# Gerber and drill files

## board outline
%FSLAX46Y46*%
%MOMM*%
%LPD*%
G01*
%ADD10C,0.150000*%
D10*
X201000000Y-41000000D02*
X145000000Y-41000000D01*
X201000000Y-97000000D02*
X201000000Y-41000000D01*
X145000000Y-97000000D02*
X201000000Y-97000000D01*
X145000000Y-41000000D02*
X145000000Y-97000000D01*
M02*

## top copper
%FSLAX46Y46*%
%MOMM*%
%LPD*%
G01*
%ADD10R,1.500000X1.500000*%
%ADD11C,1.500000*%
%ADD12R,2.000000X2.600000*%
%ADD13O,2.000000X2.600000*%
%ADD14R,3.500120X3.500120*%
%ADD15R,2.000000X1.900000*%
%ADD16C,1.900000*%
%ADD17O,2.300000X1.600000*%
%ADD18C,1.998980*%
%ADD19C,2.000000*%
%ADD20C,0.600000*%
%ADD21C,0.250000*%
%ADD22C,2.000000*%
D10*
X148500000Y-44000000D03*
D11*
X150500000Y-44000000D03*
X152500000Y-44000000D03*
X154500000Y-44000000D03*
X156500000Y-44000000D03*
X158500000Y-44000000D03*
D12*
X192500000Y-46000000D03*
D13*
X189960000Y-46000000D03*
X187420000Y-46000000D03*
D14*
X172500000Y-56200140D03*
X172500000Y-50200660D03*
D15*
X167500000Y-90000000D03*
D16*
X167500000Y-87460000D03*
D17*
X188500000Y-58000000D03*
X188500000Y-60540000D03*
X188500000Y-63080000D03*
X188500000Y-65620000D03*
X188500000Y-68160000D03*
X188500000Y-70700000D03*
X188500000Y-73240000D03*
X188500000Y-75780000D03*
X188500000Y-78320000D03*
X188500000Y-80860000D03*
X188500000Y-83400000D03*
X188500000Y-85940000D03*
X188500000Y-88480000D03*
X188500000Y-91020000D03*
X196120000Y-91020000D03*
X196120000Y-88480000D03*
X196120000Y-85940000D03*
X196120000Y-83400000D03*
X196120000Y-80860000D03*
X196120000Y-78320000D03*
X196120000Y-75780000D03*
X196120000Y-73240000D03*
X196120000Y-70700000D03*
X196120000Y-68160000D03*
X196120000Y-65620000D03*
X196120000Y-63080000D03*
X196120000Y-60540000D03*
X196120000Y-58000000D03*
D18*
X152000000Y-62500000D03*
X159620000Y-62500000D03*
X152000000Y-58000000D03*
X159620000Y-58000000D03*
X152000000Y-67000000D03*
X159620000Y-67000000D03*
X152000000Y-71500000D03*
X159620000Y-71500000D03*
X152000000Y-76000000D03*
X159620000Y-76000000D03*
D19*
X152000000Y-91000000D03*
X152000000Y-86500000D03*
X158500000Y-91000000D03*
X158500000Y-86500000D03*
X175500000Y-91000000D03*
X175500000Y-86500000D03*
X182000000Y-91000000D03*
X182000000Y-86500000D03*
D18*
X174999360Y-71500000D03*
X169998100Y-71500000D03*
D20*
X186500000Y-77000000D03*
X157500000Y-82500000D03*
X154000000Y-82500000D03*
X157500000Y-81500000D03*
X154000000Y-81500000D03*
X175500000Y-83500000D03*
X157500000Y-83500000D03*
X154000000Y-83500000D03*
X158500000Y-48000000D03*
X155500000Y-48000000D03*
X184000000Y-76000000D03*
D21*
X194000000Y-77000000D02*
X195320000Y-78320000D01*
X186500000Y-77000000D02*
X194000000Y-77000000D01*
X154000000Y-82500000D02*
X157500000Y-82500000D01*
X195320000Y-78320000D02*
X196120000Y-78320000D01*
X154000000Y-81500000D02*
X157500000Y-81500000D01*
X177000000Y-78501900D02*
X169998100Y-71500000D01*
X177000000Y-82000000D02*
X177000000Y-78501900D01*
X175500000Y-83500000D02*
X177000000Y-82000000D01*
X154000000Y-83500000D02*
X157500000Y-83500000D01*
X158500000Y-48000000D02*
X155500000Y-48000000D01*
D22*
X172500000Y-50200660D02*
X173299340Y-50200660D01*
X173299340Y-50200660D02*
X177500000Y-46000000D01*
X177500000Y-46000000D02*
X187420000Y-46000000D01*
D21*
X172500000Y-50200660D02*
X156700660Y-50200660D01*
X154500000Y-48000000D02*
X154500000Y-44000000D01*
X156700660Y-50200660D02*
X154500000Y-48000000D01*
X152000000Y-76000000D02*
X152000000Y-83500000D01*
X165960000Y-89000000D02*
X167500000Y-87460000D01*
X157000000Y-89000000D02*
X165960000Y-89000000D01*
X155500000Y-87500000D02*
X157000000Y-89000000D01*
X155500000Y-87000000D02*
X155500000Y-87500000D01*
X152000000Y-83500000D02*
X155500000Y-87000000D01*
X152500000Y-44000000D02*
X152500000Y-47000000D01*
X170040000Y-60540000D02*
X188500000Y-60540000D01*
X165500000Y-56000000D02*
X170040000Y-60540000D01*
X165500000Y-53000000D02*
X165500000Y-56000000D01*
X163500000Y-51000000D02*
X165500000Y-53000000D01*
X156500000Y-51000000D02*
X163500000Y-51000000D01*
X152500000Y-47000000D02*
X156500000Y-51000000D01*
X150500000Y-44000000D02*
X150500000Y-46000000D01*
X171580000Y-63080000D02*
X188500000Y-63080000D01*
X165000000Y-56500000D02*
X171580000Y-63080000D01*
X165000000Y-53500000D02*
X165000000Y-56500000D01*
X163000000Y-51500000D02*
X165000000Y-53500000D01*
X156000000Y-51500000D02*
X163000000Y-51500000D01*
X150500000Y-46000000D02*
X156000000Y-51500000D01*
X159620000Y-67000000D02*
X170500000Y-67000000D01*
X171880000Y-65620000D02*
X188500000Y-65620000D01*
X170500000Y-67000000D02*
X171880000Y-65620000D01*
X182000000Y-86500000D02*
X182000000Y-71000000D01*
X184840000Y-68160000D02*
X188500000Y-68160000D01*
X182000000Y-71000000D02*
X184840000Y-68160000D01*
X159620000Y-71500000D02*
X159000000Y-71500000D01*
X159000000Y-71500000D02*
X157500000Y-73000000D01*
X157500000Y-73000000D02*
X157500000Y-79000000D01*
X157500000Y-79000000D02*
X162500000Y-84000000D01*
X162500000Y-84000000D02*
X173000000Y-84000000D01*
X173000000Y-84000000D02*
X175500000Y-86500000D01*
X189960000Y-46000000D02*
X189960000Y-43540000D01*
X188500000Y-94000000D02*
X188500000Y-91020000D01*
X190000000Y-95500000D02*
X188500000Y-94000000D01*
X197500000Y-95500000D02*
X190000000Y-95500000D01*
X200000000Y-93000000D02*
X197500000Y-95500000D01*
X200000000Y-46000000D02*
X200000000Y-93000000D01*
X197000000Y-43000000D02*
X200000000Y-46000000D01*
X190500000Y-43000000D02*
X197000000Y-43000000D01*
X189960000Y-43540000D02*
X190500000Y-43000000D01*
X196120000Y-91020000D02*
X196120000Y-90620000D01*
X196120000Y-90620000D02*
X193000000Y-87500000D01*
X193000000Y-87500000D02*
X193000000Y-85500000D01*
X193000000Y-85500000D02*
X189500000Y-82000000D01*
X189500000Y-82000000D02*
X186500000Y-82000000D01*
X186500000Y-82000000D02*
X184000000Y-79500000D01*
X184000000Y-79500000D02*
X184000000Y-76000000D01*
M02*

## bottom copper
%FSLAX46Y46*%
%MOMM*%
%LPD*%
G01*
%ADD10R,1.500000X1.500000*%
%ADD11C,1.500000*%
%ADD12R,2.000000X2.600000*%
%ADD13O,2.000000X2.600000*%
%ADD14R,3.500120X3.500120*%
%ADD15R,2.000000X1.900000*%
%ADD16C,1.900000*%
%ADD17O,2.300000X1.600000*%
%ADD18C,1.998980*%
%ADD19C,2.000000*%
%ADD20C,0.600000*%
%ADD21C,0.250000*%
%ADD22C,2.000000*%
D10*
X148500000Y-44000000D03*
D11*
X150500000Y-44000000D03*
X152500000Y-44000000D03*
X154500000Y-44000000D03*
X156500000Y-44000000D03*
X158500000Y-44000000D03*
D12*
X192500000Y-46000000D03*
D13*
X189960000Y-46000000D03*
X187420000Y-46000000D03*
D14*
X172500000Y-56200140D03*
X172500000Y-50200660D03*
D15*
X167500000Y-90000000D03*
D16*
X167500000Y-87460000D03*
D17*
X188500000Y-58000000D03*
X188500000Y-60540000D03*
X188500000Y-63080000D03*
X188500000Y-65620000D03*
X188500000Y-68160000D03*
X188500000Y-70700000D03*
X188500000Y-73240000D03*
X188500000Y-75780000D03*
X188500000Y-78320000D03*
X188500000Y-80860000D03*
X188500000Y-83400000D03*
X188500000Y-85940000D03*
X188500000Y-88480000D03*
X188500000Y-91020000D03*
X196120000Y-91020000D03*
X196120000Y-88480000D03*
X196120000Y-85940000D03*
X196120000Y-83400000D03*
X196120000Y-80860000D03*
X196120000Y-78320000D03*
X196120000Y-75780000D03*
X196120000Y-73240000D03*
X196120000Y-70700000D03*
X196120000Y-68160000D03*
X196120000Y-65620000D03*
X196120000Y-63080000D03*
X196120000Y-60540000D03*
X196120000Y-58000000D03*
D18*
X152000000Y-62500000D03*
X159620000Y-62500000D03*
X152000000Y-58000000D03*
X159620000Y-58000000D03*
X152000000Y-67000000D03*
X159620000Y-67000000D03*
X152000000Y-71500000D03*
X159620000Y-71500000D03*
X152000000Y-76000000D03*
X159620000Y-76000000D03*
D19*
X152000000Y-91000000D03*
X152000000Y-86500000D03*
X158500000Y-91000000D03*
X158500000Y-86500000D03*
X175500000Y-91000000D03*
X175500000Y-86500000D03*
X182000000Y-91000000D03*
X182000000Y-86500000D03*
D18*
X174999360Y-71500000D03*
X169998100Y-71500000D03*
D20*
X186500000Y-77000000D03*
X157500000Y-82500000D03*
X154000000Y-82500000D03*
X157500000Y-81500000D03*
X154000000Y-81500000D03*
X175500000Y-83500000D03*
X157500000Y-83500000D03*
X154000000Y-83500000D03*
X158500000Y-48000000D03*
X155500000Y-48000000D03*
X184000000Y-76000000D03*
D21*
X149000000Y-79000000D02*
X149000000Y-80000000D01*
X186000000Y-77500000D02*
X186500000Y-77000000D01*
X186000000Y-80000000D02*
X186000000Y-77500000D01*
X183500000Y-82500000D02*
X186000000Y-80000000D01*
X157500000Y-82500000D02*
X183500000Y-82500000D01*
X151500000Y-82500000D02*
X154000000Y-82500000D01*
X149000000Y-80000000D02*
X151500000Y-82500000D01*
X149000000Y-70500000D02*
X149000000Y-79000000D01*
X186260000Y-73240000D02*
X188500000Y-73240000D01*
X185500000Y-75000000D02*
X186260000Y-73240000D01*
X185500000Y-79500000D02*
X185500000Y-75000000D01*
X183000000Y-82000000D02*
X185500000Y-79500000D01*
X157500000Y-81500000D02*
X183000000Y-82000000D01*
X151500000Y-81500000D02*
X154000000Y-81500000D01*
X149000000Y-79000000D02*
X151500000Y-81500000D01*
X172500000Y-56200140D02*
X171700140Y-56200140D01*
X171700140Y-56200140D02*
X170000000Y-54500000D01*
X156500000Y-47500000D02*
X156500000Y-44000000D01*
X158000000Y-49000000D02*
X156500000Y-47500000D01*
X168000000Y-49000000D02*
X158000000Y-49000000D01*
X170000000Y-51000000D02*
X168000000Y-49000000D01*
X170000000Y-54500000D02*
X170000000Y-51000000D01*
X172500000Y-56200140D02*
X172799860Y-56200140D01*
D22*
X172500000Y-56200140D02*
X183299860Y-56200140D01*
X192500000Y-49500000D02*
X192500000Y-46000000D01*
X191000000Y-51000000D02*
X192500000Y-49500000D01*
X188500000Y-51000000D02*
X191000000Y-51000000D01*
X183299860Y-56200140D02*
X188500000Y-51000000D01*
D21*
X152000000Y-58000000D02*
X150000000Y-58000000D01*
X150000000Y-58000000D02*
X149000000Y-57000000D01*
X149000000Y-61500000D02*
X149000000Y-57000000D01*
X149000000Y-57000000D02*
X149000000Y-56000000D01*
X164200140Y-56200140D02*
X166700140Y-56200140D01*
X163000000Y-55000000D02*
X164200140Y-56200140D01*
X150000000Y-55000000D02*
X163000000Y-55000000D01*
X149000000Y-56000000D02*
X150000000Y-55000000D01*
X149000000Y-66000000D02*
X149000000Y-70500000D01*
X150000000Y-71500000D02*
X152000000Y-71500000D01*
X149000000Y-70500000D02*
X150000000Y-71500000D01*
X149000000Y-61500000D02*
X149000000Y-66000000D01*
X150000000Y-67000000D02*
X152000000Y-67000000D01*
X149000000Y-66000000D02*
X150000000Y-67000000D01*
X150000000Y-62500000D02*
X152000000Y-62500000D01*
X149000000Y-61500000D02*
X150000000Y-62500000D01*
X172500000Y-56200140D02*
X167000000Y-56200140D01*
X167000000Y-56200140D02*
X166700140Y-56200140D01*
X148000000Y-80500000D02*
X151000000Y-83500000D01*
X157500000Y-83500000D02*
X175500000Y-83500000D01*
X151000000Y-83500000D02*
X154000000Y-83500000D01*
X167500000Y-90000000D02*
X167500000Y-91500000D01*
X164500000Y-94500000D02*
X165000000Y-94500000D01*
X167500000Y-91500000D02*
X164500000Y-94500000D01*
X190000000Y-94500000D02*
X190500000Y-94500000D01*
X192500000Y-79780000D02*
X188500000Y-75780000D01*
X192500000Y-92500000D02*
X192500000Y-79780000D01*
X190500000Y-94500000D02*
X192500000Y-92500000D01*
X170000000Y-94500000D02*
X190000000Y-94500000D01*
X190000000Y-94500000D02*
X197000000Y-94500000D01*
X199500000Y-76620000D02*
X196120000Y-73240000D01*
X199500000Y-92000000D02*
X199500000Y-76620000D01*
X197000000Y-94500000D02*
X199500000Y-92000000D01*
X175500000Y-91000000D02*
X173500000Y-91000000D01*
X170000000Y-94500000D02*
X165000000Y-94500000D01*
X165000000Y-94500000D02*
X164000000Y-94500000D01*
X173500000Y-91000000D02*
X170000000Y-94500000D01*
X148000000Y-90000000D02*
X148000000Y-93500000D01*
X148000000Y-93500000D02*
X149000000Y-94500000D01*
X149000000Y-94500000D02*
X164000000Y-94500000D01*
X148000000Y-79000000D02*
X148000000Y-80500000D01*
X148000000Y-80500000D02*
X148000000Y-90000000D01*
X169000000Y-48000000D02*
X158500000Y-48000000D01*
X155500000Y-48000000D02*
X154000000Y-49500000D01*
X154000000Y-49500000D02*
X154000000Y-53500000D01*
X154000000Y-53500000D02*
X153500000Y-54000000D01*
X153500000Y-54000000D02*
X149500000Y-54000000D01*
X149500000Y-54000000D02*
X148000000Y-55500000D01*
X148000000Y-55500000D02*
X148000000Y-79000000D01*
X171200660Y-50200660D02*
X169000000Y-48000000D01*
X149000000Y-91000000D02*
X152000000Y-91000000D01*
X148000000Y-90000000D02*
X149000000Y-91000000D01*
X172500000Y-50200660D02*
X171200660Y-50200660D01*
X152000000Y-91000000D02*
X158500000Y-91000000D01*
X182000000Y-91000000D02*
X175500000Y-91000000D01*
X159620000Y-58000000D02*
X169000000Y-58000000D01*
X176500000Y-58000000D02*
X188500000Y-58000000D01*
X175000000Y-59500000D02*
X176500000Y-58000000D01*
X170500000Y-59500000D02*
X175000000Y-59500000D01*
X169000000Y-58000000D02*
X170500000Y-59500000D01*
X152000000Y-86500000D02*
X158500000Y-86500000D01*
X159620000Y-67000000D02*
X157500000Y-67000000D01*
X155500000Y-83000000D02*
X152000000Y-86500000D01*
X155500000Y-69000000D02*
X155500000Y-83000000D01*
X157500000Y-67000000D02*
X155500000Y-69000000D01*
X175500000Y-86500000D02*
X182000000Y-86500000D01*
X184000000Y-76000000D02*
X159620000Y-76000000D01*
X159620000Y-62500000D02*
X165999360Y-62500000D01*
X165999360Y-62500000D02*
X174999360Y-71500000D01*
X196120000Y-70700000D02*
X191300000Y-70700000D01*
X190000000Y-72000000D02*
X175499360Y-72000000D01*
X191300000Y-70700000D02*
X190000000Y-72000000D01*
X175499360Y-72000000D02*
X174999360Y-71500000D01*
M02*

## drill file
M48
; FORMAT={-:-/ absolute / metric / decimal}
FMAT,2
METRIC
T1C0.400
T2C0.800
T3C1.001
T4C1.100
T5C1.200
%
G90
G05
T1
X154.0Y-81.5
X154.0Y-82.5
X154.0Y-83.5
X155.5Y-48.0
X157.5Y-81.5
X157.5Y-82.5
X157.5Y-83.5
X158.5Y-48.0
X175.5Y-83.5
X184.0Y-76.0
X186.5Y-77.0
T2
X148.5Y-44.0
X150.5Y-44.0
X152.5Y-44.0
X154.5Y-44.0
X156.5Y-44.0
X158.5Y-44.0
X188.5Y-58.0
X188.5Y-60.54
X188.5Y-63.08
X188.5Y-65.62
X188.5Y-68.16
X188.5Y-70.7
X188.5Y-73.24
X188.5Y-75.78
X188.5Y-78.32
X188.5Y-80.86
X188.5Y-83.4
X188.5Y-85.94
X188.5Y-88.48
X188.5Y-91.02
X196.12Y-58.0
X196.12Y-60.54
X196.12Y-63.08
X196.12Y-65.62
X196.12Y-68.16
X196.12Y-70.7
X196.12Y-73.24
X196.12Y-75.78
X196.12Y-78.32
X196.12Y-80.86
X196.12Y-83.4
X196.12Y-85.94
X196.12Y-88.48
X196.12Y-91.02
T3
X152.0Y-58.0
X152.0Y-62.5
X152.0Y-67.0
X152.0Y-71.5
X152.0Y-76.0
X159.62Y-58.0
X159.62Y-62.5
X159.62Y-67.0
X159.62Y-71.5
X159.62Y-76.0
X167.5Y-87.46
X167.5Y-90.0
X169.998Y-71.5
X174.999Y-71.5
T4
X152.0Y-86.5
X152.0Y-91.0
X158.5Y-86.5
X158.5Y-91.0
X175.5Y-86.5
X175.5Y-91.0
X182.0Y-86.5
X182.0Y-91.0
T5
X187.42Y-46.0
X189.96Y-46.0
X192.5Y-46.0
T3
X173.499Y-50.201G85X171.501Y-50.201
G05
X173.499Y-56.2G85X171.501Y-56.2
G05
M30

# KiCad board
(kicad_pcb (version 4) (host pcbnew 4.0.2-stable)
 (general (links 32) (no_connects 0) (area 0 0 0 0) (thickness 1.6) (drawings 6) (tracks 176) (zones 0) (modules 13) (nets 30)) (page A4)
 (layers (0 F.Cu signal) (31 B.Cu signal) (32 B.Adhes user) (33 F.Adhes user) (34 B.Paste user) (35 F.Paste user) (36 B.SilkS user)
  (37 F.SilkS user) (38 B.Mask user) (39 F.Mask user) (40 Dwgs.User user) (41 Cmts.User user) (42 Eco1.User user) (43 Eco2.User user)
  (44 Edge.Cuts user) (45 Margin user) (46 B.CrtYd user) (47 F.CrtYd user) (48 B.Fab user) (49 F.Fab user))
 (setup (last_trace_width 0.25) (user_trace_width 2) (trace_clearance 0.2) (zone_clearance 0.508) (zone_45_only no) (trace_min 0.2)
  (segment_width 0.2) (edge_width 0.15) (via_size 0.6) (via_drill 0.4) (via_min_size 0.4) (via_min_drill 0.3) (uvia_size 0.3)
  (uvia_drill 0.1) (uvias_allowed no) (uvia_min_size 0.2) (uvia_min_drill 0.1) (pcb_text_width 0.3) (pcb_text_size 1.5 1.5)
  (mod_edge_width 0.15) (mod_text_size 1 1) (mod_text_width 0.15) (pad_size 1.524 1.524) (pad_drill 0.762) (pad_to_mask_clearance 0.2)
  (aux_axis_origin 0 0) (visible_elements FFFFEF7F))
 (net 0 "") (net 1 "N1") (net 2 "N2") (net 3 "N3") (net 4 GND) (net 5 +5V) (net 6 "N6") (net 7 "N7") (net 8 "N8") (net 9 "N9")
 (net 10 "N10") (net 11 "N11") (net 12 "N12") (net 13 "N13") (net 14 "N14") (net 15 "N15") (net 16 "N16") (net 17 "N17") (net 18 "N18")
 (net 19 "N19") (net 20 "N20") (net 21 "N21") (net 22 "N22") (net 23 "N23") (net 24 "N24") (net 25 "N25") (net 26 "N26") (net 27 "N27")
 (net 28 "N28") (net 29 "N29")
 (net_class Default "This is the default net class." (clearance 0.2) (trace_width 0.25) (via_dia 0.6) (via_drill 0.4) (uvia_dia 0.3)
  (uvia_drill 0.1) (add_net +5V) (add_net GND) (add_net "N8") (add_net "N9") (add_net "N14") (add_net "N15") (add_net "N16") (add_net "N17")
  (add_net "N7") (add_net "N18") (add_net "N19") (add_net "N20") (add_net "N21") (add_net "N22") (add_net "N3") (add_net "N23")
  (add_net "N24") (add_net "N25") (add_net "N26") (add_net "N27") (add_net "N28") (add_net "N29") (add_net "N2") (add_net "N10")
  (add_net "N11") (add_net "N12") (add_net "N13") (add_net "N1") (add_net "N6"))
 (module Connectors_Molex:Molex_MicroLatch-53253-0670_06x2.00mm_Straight (layer F.Cu) (at 148.5 44)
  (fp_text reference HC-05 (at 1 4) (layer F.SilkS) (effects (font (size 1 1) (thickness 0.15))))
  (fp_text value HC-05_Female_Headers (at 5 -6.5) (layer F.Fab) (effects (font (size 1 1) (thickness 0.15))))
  (pad 1 thru_hole rect (at 0 0) (size 1.5 1.5) (drill 0.8) (layers *.Cu *.Mask) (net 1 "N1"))
  (pad 2 thru_hole circle (at 2 0) (size 1.5 1.5) (drill 0.8) (layers *.Cu *.Mask) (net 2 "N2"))
  (pad 3 thru_hole circle (at 4 0) (size 1.5 1.5) (drill 0.8) (layers *.Cu *.Mask) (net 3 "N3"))
  (pad 4 thru_hole circle (at 6 0) (size 1.5 1.5) (drill 0.8) (layers *.Cu *.Mask) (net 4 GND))
  (pad 5 thru_hole circle (at 8 0) (size 1.5 1.5) (drill 0.8) (layers *.Cu *.Mask) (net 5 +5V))
  (pad 6 thru_hole circle (at 10 0) (size 1.5 1.5) (drill 0.8) (layers *.Cu *.Mask) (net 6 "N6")))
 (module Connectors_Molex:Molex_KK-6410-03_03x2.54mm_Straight (layer F.Cu) (at 192.5 46 180)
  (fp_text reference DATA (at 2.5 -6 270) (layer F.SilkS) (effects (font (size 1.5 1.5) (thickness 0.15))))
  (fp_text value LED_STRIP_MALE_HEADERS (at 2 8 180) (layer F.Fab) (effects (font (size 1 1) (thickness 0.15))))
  (pad 1 thru_hole rect (at 0 0 180) (size 2 2.6) (drill 1.2) (layers *.Cu *.Mask F.SilkS) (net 5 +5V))
  (pad 2 thru_hole oval (at 2.54 0 180) (size 2 2.6) (drill 1.2) (layers *.Cu *.Mask F.SilkS) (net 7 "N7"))
  (pad 3 thru_hole oval (at 5.08 0 180) (size 2 2.6) (drill 1.2) (layers *.Cu *.Mask F.SilkS) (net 4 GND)))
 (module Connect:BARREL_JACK (layer F.Cu) (at 172.5 50 270)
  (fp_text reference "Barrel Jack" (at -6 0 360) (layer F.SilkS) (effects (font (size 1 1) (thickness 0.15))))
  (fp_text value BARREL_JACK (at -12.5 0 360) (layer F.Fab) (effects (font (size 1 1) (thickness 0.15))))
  (pad 1 thru_hole rect (at 6.20014 0 270) (size 3.50012 3.50012) (drill oval 1.00076 2.99974) (layers *.Cu *.Mask F.SilkS) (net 5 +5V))
  (pad 2 thru_hole rect (at 0.20066 0 270) (size 3.50012 3.50012) (drill oval 1.00076 2.99974) (layers *.Cu *.Mask F.SilkS) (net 4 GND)))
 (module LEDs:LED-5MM (layer F.Cu) (at 167.5 90 90)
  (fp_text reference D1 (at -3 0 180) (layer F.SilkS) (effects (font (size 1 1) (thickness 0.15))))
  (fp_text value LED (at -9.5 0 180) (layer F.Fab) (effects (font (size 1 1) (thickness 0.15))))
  (pad 1 thru_hole rect (at 0 0 180) (size 2 1.9) (drill 1.00076) (layers *.Cu *.Mask F.SilkS) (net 4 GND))
  (pad 2 thru_hole circle (at 2.54 0 90) (size 1.9 1.9) (drill 1.00076) (layers *.Cu *.Mask F.SilkS) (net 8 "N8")))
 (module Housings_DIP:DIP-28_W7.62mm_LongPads (layer F.Cu) (at 188.5 58)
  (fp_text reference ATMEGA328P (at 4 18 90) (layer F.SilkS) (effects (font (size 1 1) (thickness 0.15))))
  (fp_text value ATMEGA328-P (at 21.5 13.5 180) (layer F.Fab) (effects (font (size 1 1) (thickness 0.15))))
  (pad 1 thru_hole oval (at 0 0) (size 2.3 1.6) (drill 0.8) (layers *.Cu *.Mask F.SilkS) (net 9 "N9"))
  (pad 2 thru_hole oval (at 0 2.54) (size 2.3 1.6) (drill 0.8) (layers *.Cu *.Mask F.SilkS) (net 3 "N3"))
  (pad 3 thru_hole oval (at 0 5.08) (size 2.3 1.6) (drill 0.8) (layers *.Cu *.Mask F.SilkS) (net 2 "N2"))
  (pad 4 thru_hole oval (at 0 7.62) (size 2.3 1.6) (drill 0.8) (layers *.Cu *.Mask F.SilkS) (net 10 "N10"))
  (pad 5 thru_hole oval (at 0 10.16) (size 2.3 1.6) (drill 0.8) (layers *.Cu *.Mask F.SilkS) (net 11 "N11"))
  (pad 6 thru_hole oval (at 0 12.7) (size 2.3 1.6) (drill 0.8) (layers *.Cu *.Mask F.SilkS) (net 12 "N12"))
  (pad 7 thru_hole oval (at 0 15.24) (size 2.3 1.6) (drill 0.8) (layers *.Cu *.Mask F.SilkS) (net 5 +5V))
  (pad 8 thru_hole oval (at 0 17.78) (size 2.3 1.6) (drill 0.8) (layers *.Cu *.Mask F.SilkS) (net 4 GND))
  (pad 9 thru_hole oval (at 0 20.32) (size 2.3 1.6) (drill 0.8) (layers *.Cu *.Mask F.SilkS) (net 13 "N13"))
  (pad 10 thru_hole oval (at 0 22.86) (size 2.3 1.6) (drill 0.8) (layers *.Cu *.Mask F.SilkS) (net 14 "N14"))
  (pad 11 thru_hole oval (at 0 25.4) (size 2.3 1.6) (drill 0.8) (layers *.Cu *.Mask F.SilkS) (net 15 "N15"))
  (pad 12 thru_hole oval (at 0 27.94) (size 2.3 1.6) (drill 0.8) (layers *.Cu *.Mask F.SilkS) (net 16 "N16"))
  (pad 13 thru_hole oval (at 0 30.48) (size 2.3 1.6) (drill 0.8) (layers *.Cu *.Mask F.SilkS) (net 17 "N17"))
  (pad 14 thru_hole oval (at 0 33.02) (size 2.3 1.6) (drill 0.8) (layers *.Cu *.Mask F.SilkS) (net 7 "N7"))
  (pad 15 thru_hole oval (at 7.62 33.02) (size 2.3 1.6) (drill 0.8) (layers *.Cu *.Mask F.SilkS) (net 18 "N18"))
  (pad 16 thru_hole oval (at 7.62 30.48) (size 2.3 1.6) (drill 0.8) (layers *.Cu *.Mask F.SilkS) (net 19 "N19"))
  (pad 17 thru_hole oval (at 7.62 27.94) (size 2.3 1.6) (drill 0.8) (layers *.Cu *.Mask F.SilkS) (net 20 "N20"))
  (pad 18 thru_hole oval (at 7.62 25.4) (size 2.3 1.6) (drill 0.8) (layers *.Cu *.Mask F.SilkS) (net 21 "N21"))
  (pad 19 thru_hole oval (at 7.62 22.86) (size 2.3 1.6) (drill 0.8) (layers *.Cu *.Mask F.SilkS) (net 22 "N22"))
  (pad 20 thru_hole oval (at 7.62 20.32) (size 2.3 1.6) (drill 0.8) (layers *.Cu *.Mask F.SilkS) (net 5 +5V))
  (pad 21 thru_hole oval (at 7.62 17.78) (size 2.3 1.6) (drill 0.8) (layers *.Cu *.Mask F.SilkS) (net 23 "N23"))
  (pad 22 thru_hole oval (at 7.62 15.24) (size 2.3 1.6) (drill 0.8) (layers *.Cu *.Mask F.SilkS) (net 4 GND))
  (pad 23 thru_hole oval (at 7.62 12.7) (size 2.3 1.6) (drill 0.8) (layers *.Cu *.Mask F.SilkS) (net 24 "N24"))
  (pad 24 thru_hole oval (at 7.62 10.16) (size 2.3 1.6) (drill 0.8) (layers *.Cu *.Mask F.SilkS) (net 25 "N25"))
  (pad 25 thru_hole oval (at 7.62 7.62) (size 2.3 1.6) (drill 0.8) (layers *.Cu *.Mask F.SilkS) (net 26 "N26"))
  (pad 26 thru_hole oval (at 7.62 5.08) (size 2.3 1.6) (drill 0.8) (layers *.Cu *.Mask F.SilkS) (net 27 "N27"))
  (pad 27 thru_hole oval (at 7.62 2.54) (size 2.3 1.6) (drill 0.8) (layers *.Cu *.Mask F.SilkS) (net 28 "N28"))
  (pad 28 thru_hole oval (at 7.62 0) (size 2.3 1.6) (drill 0.8) (layers *.Cu *.Mask F.SilkS) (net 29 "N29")))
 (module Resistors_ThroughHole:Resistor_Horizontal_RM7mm (layer F.Cu) (at 152 62.5)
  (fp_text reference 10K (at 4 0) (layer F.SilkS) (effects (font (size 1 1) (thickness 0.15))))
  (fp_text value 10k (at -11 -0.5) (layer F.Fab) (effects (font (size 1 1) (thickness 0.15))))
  (pad 1 thru_hole circle (at 0 0) (size 1.99898 1.99898) (drill 1.00076) (layers *.Cu *.SilkS *.Mask) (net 5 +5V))
  (pad 2 thru_hole circle (at 7.62 0) (size 1.99898 1.99898) (drill 1.00076) (layers *.Cu *.SilkS *.Mask) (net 24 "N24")))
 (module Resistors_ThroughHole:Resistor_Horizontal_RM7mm (layer F.Cu) (at 152 58)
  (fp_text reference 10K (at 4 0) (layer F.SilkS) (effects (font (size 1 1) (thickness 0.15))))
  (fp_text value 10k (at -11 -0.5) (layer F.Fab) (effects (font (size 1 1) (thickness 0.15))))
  (pad 1 thru_hole circle (at 0 0) (size 1.99898 1.99898) (drill 1.00076) (layers *.Cu *.SilkS *.Mask) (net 5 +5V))
  (pad 2 thru_hole circle (at 7.62 0) (size 1.99898 1.99898) (drill 1.00076) (layers *.Cu *.SilkS *.Mask) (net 9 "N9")))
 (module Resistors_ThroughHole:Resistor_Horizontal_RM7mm (layer F.Cu) (at 152 67)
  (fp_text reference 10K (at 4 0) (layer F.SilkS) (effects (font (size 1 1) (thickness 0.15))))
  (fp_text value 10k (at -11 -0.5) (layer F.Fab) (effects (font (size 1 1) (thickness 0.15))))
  (pad 1 thru_hole circle (at 0 0) (size 1.99898 1.99898) (drill 1.00076) (layers *.Cu *.SilkS *.Mask) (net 5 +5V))
  (pad 2 thru_hole circle (at 7.62 0) (size 1.99898 1.99898) (drill 1.00076) (layers *.Cu *.SilkS *.Mask) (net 10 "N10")))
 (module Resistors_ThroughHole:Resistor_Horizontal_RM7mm (layer F.Cu) (at 152 71.5)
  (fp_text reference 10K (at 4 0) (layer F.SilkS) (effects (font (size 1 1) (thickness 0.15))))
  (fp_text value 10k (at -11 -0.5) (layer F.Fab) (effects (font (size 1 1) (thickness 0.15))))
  (pad 1 thru_hole circle (at 0 0) (size 1.99898 1.99898) (drill 1.00076) (layers *.Cu *.SilkS *.Mask) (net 5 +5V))
  (pad 2 thru_hole circle (at 7.62 0) (size 1.99898 1.99898) (drill 1.00076) (layers *.Cu *.SilkS *.Mask) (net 11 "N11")))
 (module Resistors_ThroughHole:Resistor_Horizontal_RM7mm (layer F.Cu) (at 152 76)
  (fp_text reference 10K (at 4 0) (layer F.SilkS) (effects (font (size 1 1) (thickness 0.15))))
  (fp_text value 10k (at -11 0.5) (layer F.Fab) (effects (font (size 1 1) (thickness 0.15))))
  (pad 1 thru_hole circle (at 0 0) (size 1.99898 1.99898) (drill 1.00076) (layers *.Cu *.SilkS *.Mask) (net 8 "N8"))
  (pad 2 thru_hole circle (at 7.62 0) (size 1.99898 1.99898) (drill 1.00076) (layers *.Cu *.SilkS *.Mask) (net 18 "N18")))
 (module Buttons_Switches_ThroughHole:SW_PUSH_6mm (layer F.Cu) (at 152 86.5)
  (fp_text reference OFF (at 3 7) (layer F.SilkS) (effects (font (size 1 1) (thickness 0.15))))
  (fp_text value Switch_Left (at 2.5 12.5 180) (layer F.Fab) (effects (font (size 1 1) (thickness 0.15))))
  (pad 2 thru_hole circle (at 0 4.5 90) (size 2 2) (drill 1.1) (layers *.Cu *.Mask) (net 4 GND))
  (pad 1 thru_hole circle (at 0 0 90) (size 2 2) (drill 1.1) (layers *.Cu *.Mask) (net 10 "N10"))
  (pad 2 thru_hole circle (at 6.5 4.5 90) (size 2 2) (drill 1.1) (layers *.Cu *.Mask) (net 4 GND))
  (pad 1 thru_hole circle (at 6.5 0 90) (size 2 2) (drill 1.1) (layers *.Cu *.Mask) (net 10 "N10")))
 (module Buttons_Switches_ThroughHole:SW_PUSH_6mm (layer F.Cu) (at 175.5 86.5)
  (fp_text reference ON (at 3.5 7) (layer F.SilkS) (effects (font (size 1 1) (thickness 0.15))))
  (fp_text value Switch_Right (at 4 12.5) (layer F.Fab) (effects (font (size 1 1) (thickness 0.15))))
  (pad 2 thru_hole circle (at 0 4.5 90) (size 2 2) (drill 1.1) (layers *.Cu *.Mask) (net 4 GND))
  (pad 1 thru_hole circle (at 0 0 90) (size 2 2) (drill 1.1) (layers *.Cu *.Mask) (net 11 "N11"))
  (pad 2 thru_hole circle (at 6.5 4.5 90) (size 2 2) (drill 1.1) (layers *.Cu *.Mask) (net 4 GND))
  (pad 1 thru_hole circle (at 6.5 0 90) (size 2 2) (drill 1.1) (layers *.Cu *.Mask) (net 11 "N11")))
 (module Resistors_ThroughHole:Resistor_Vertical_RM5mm (layer F.Cu) (at 172.5 71.5 180)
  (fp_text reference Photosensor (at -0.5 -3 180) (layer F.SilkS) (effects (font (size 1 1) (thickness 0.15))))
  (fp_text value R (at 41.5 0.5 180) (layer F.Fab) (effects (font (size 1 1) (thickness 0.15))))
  (pad 1 thru_hole circle (at -2.49936 0 180) (size 1.99898 1.99898) (drill 1.00076) (layers *.Cu *.SilkS *.Mask) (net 24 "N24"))
  (pad 2 thru_hole circle (at 2.5019 0 180) (size 1.99898 1.99898) (drill 1.00076) (layers *.Cu *.SilkS *.Mask) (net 4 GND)))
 (gr_line (start 201 41) (end 145 41) (angle 90) (layer Edge.Cuts) (width 0.15))
 (gr_line (start 201 97) (end 201 41) (angle 90) (layer Edge.Cuts) (width 0.15))
 (gr_line (start 145 97) (end 201 97) (angle 90) (layer Edge.Cuts) (width 0.15))
 (gr_line (start 145 41) (end 145 97) (angle 90) (layer Edge.Cuts) (width 0.15))
 (segment (start 149 79) (end 149 80) (width 0.25) (layer B.Cu) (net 5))
 (segment (start 194 77) (end 195.32 78.32) (width 0.25) (layer F.Cu) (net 5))
 (segment (start 186.5 77) (end 194 77) (width 0.25) (layer F.Cu) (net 5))
 (via (at 186.5 77) (size 0.6) (drill 0.4) (layers F.Cu B.Cu) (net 5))
 (segment (start 186 77.5) (end 186.5 77) (width 0.25) (layer B.Cu) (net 5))
 (segment (start 186 80) (end 186 77.5) (width 0.25) (layer B.Cu) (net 5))
 (segment (start 183.5 82.5) (end 186 80) (width 0.25) (layer B.Cu) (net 5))
 (segment (start 157.5 82.5) (end 183.5 82.5) (width 0.25) (layer B.Cu) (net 5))
 (via (at 157.5 82.5) (size 0.6) (drill 0.4) (layers F.Cu B.Cu) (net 5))
 (segment (start 154 82.5) (end 157.5 82.5) (width 0.25) (layer F.Cu) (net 5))
 (via (at 154 82.5) (size 0.6) (drill 0.4) (layers F.Cu B.Cu) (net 5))
 (segment (start 151.5 82.5) (end 154 82.5) (width 0.25) (layer B.Cu) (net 5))
 (segment (start 149 80) (end 151.5 82.5) (width 0.25) (layer B.Cu) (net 5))
 (segment (start 195.32 78.32) (end 196.12 78.32) (width 0.25) (layer F.Cu) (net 5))
 (segment (start 149 70.5) (end 149 79) (width 0.25) (layer B.Cu) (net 5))
 (segment (start 186.26 73.24) (end 188.5 73.24) (width 0.25) (layer B.Cu) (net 5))
 (segment (start 185.5 75) (end 186.26 73.24) (width 0.25) (layer B.Cu) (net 5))
 (segment (start 185.5 79.5) (end 185.5 75) (width 0.25) (layer B.Cu) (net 5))
 (segment (start 183 82) (end 185.5 79.5) (width 0.25) (layer B.Cu) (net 5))
 (segment (start 157.5 81.5) (end 183 82) (width 0.25) (layer B.Cu) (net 5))
 (via (at 157.5 81.5) (size 0.6) (drill 0.4) (layers F.Cu B.Cu) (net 5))
 (segment (start 154 81.5) (end 157.5 81.5) (width 0.25) (layer F.Cu) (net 5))
 (via (at 154 81.5) (size 0.6) (drill 0.4) (layers F.Cu B.Cu) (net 5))
 (segment (start 151.5 81.5) (end 154 81.5) (width 0.25) (layer B.Cu) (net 5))
 (segment (start 149 79) (end 151.5 81.5) (width 0.25) (layer B.Cu) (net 5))
 (segment (start 172.5 56.20014) (end 171.70014 56.20014) (width 0.25) (layer B.Cu) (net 5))
 (segment (start 171.70014 56.20014) (end 170 54.5) (width 0.25) (layer B.Cu) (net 5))
 (segment (start 156.5 47.5) (end 156.5 44) (width 0.25) (layer B.Cu) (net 5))
 (segment (start 158 49) (end 156.5 47.5) (width 0.25) (layer B.Cu) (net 5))
 (segment (start 168 49) (end 158 49) (width 0.25) (layer B.Cu) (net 5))
 (segment (start 170 51) (end 168 49) (width 0.25) (layer B.Cu) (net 5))
 (segment (start 170 54.5) (end 170 51) (width 0.25) (layer B.Cu) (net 5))
 (segment (start 172.5 56.20014) (end 172.79986 56.20014) (width 0.25) (layer B.Cu) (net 5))
 (segment (start 172.5 56.20014) (end 183.29986 56.20014) (width 2) (layer B.Cu) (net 5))
 (segment (start 192.5 49.5) (end 192.5 46) (width 2) (layer B.Cu) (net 5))
 (segment (start 191 51) (end 192.5 49.5) (width 2) (layer B.Cu) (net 5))
 (segment (start 188.5 51) (end 191 51) (width 2) (layer B.Cu) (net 5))
 (segment (start 183.29986 56.20014) (end 188.5 51) (width 2) (layer B.Cu) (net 5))
 (segment (start 152 58) (end 150 58) (width 0.25) (layer B.Cu) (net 5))
 (segment (start 150 58) (end 149 57) (width 0.25) (layer B.Cu) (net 5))
 (segment (start 149 61.5) (end 149 57) (width 0.25) (layer B.Cu) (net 5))
 (segment (start 149 57) (end 149 56) (width 0.25) (layer B.Cu) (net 5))
 (segment (start 164.20014 56.20014) (end 166.70014 56.20014) (width 0.25) (layer B.Cu) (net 5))
 (segment (start 163 55) (end 164.20014 56.20014) (width 0.25) (layer B.Cu) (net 5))
 (segment (start 150 55) (end 163 55) (width 0.25) (layer B.Cu) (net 5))
 (segment (start 149 56) (end 150 55) (width 0.25) (layer B.Cu) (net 5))
 (segment (start 149 66) (end 149 70.5) (width 0.25) (layer B.Cu) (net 5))
 (segment (start 150 71.5) (end 152 71.5) (width 0.25) (layer B.Cu) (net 5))
 (segment (start 149 70.5) (end 150 71.5) (width 0.25) (layer B.Cu) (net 5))
 (segment (start 149 61.5) (end 149 66) (width 0.25) (layer B.Cu) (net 5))
 (segment (start 150 67) (end 152 67) (width 0.25) (layer B.Cu) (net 5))
 (segment (start 149 66) (end 150 67) (width 0.25) (layer B.Cu) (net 5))
 (segment (start 150 62.5) (end 152 62.5) (width 0.25) (layer B.Cu) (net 5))
 (segment (start 149 61.5) (end 150 62.5) (width 0.25) (layer B.Cu) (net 5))
 (segment (start 172.5 56.20014) (end 167 56.20014) (width 0.25) (layer B.Cu) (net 5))
 (segment (start 167 56.20014) (end 166.70014 56.20014) (width 0.25) (layer B.Cu) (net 5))
 (segment (start 148 80.5) (end 151 83.5) (width 0.25) (layer B.Cu) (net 4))
 (segment (start 177 78.5019) (end 169.9981 71.5) (width 0.25) (layer F.Cu) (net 4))
 (segment (start 177 82) (end 177 78.5019) (width 0.25) (layer F.Cu) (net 4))
 (segment (start 175.5 83.5) (end 177 82) (width 0.25) (layer F.Cu) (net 4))
 (via (at 175.5 83.5) (size 0.6) (drill 0.4) (layers F.Cu B.Cu) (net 4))
 (segment (start 157.5 83.5) (end 175.5 83.5) (width 0.25) (layer B.Cu) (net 4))
 (via (at 157.5 83.5) (size 0.6) (drill 0.4) (layers F.Cu B.Cu) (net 4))
 (segment (start 154 83.5) (end 157.5 83.5) (width 0.25) (layer F.Cu) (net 4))
 (via (at 154 83.5) (size 0.6) (drill 0.4) (layers F.Cu B.Cu) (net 4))
 (segment (start 151 83.5) (end 154 83.5) (width 0.25) (layer B.Cu) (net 4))
 (segment (start 167.5 90) (end 167.5 91.5) (width 0.25) (layer B.Cu) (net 4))
 (segment (start 164.5 94.5) (end 165 94.5) (width 0.25) (layer B.Cu) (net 4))
 (segment (start 167.5 91.5) (end 164.5 94.5) (width 0.25) (layer B.Cu) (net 4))
 (segment (start 190 94.5) (end 190.5 94.5) (width 0.25) (layer B.Cu) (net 4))
 (segment (start 192.5 79.78) (end 188.5 75.78) (width 0.25) (layer B.Cu) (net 4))
 (segment (start 192.5 92.5) (end 192.5 79.78) (width 0.25) (layer B.Cu) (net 4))
 (segment (start 190.5 94.5) (end 192.5 92.5) (width 0.25) (layer B.Cu) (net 4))
 (segment (start 170 94.5) (end 190 94.5) (width 0.25) (layer B.Cu) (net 4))
 (segment (start 190 94.5) (end 197 94.5) (width 0.25) (layer B.Cu) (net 4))
 (segment (start 199.5 76.62) (end 196.12 73.24) (width 0.25) (layer B.Cu) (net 4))
 (segment (start 199.5 92) (end 199.5 76.62) (width 0.25) (layer B.Cu) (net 4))
 (segment (start 197 94.5) (end 199.5 92) (width 0.25) (layer B.Cu) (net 4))
 (segment (start 175.5 91) (end 173.5 91) (width 0.25) (layer B.Cu) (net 4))
 (segment (start 170 94.5) (end 165 94.5) (width 0.25) (layer B.Cu) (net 4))
 (segment (start 165 94.5) (end 164 94.5) (width 0.25) (layer B.Cu) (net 4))
 (segment (start 173.5 91) (end 170 94.5) (width 0.25) (layer B.Cu) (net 4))
 (segment (start 148 90) (end 148 93.5) (width 0.25) (layer B.Cu) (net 4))
 (segment (start 148 93.5) (end 149 94.5) (width 0.25) (layer B.Cu) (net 4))
 (segment (start 149 94.5) (end 164 94.5) (width 0.25) (layer B.Cu) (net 4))
 (segment (start 148 79) (end 148 80.5) (width 0.25) (layer B.Cu) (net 4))
 (segment (start 148 80.5) (end 148 90) (width 0.25) (layer B.Cu) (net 4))
 (segment (start 169 48) (end 158.5 48) (width 0.25) (layer B.Cu) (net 4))
 (via (at 158.5 48) (size 0.6) (drill 0.4) (layers F.Cu B.Cu) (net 4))
 (segment (start 158.5 48) (end 155.5 48) (width 0.25) (layer F.Cu) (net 4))
 (via (at 155.5 48) (size 0.6) (drill 0.4) (layers F.Cu B.Cu) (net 4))
 (segment (start 155.5 48) (end 154 49.5) (width 0.25) (layer B.Cu) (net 4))
 (segment (start 154 49.5) (end 154 53.5) (width 0.25) (layer B.Cu) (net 4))
 (segment (start 154 53.5) (end 153.5 54) (width 0.25) (layer B.Cu) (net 4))
 (segment (start 153.5 54) (end 149.5 54) (width 0.25) (layer B.Cu) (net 4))
 (segment (start 149.5 54) (end 148 55.5) (width 0.25) (layer B.Cu) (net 4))
 (segment (start 148 55.5) (end 148 79) (width 0.25) (layer B.Cu) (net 4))
 (segment (start 171.20066 50.20066) (end 169 48) (width 0.25) (layer B.Cu) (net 4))
 (segment (start 149 91) (end 152 91) (width 0.25) (layer B.Cu) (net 4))
 (segment (start 148 90) (end 149 91) (width 0.25) (layer B.Cu) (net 4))
 (segment (start 172.5 50.20066) (end 171.20066 50.20066) (width 0.25) (layer B.Cu) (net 4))
 (segment (start 152 91) (end 158.5 91) (width 0.25) (layer B.Cu) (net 4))
 (segment (start 182 91) (end 175.5 91) (width 0.25) (layer B.Cu) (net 4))
 (segment (start 172.5 50.20066) (end 173.29934 50.20066) (width 2) (layer F.Cu) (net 4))
 (segment (start 173.29934 50.20066) (end 177.5 46) (width 2) (layer F.Cu) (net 4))
 (segment (start 177.5 46) (end 187.42 46) (width 2) (layer F.Cu) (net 4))
 (segment (start 172.5 50.20066) (end 156.70066 50.20066) (width 0.25) (layer F.Cu) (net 4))
 (segment (start 154.5 48) (end 154.5 44) (width 0.25) (layer F.Cu) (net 4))
 (segment (start 156.70066 50.20066) (end 154.5 48) (width 0.25) (layer F.Cu) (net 4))
 (segment (start 152 76) (end 152 83.5) (width 0.25) (layer F.Cu) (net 8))
 (segment (start 165.96 89) (end 167.5 87.46) (width 0.25) (layer F.Cu) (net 8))
 (segment (start 157 89) (end 165.96 89) (width 0.25) (layer F.Cu) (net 8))
 (segment (start 155.5 87.5) (end 157 89) (width 0.25) (layer F.Cu) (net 8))
 (segment (start 155.5 87) (end 155.5 87.5) (width 0.25) (layer F.Cu) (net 8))
 (segment (start 152 83.5) (end 155.5 87) (width 0.25) (layer F.Cu) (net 8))
 (segment (start 159.62 58) (end 169 58) (width 0.25) (layer B.Cu) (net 9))
 (segment (start 176.5 58) (end 188.5 58) (width 0.25) (layer B.Cu) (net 9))
 (segment (start 175 59.5) (end 176.5 58) (width 0.25) (layer B.Cu) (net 9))
 (segment (start 170.5 59.5) (end 175 59.5) (width 0.25) (layer B.Cu) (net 9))
 (segment (start 169 58) (end 170.5 59.5) (width 0.25) (layer B.Cu) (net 9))
 (segment (start 152.5 44) (end 152.5 47) (width 0.25) (layer F.Cu) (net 3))
 (segment (start 170.04 60.54) (end 188.5 60.54) (width 0.25) (layer F.Cu) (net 3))
 (segment (start 165.5 56) (end 170.04 60.54) (width 0.25) (layer F.Cu) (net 3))
 (segment (start 165.5 53) (end 165.5 56) (width 0.25) (layer F.Cu) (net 3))
 (segment (start 163.5 51) (end 165.5 53) (width 0.25) (layer F.Cu) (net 3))
 (segment (start 156.5 51) (end 163.5 51) (width 0.25) (layer F.Cu) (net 3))
 (segment (start 152.5 47) (end 156.5 51) (width 0.25) (layer F.Cu) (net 3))
 (segment (start 150.5 44) (end 150.5 46) (width 0.25) (layer F.Cu) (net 2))
 (segment (start 171.58 63.08) (end 188.5 63.08) (width 0.25) (layer F.Cu) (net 2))
 (segment (start 165 56.5) (end 171.58 63.08) (width 0.25) (layer F.Cu) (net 2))
 (segment (start 165 53.5) (end 165 56.5) (width 0.25) (layer F.Cu) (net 2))
 (segment (start 163 51.5) (end 165 53.5) (width 0.25) (layer F.Cu) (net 2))
 (segment (start 156 51.5) (end 163 51.5) (width 0.25) (layer F.Cu) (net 2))
 (segment (start 150.5 46) (end 156 51.5) (width 0.25) (layer F.Cu) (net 2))
 (segment (start 159.62 67) (end 170.5 67) (width 0.25) (layer F.Cu) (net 10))
 (segment (start 171.88 65.62) (end 188.5 65.62) (width 0.25) (layer F.Cu) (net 10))
 (segment (start 170.5 67) (end 171.88 65.62) (width 0.25) (layer F.Cu) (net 10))
 (segment (start 152 86.5) (end 158.5 86.5) (width 0.25) (layer B.Cu) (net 10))
 (segment (start 159.62 67) (end 157.5 67) (width 0.25) (layer B.Cu) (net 10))
 (segment (start 155.5 83) (end 152 86.5) (width 0.25) (layer B.Cu) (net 10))
 (segment (start 155.5 69) (end 155.5 83) (width 0.25) (layer B.Cu) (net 10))
 (segment (start 157.5 67) (end 155.5 69) (width 0.25) (layer B.Cu) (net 10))
 (segment (start 182 86.5) (end 182 71) (width 0.25) (layer F.Cu) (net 11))
 (segment (start 184.84 68.16) (end 188.5 68.16) (width 0.25) (layer F.Cu) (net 11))
 (segment (start 182 71) (end 184.84 68.16) (width 0.25) (layer F.Cu) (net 11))
 (segment (start 159.62 71.5) (end 159 71.5) (width 0.25) (layer F.Cu) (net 11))
 (segment (start 159 71.5) (end 157.5 73) (width 0.25) (layer F.Cu) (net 11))
 (segment (start 157.5 73) (end 157.5 79) (width 0.25) (layer F.Cu) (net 11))
 (segment (start 157.5 79) (end 162.5 84) (width 0.25) (layer F.Cu) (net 11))
 (segment (start 162.5 84) (end 173 84) (width 0.25) (layer F.Cu) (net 11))
 (segment (start 173 84) (end 175.5 86.5) (width 0.25) (layer F.Cu) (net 11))
 (segment (start 175.5 86.5) (end 182 86.5) (width 0.25) (layer B.Cu) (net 11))
 (segment (start 189.96 46) (end 189.96 43.54) (width 0.25) (layer F.Cu) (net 7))
 (segment (start 188.5 94) (end 188.5 91.02) (width 0.25) (layer F.Cu) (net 7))
 (segment (start 190 95.5) (end 188.5 94) (width 0.25) (layer F.Cu) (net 7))
 (segment (start 197.5 95.5) (end 190 95.5) (width 0.25) (layer F.Cu) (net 7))
 (segment (start 200 93) (end 197.5 95.5) (width 0.25) (layer F.Cu) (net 7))
 (segment (start 200 46) (end 200 93) (width 0.25) (layer F.Cu) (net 7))
 (segment (start 197 43) (end 200 46) (width 0.25) (layer F.Cu) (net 7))
 (segment (start 190.5 43) (end 197 43) (width 0.25) (layer F.Cu) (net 7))
 (segment (start 189.96 43.54) (end 190.5 43) (width 0.25) (layer F.Cu) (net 7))
 (segment (start 196.12 91.02) (end 196.12 90.62) (width 0.25) (layer F.Cu) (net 18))
 (segment (start 196.12 90.62) (end 193 87.5) (width 0.25) (layer F.Cu) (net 18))
 (segment (start 193 87.5) (end 193 85.5) (width 0.25) (layer F.Cu) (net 18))
 (segment (start 193 85.5) (end 189.5 82) (width 0.25) (layer F.Cu) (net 18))
 (segment (start 189.5 82) (end 186.5 82) (width 0.25) (layer F.Cu) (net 18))
 (segment (start 186.5 82) (end 184 79.5) (width 0.25) (layer F.Cu) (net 18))
 (segment (start 184 79.5) (end 184 76) (width 0.25) (layer F.Cu) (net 18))
 (via (at 184 76) (size 0.6) (drill 0.4) (layers F.Cu B.Cu) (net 18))
 (segment (start 184 76) (end 159.62 76) (width 0.25) (layer B.Cu) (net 18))
 (segment (start 159.62 62.5) (end 165.99936 62.5) (width 0.25) (layer B.Cu) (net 24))
 (segment (start 165.99936 62.5) (end 174.99936 71.5) (width 0.25) (layer B.Cu) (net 24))
 (segment (start 196.12 70.7) (end 191.3 70.7) (width 0.25) (layer B.Cu) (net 24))
 (segment (start 190 72) (end 175.49936 72) (width 0.25) (layer B.Cu) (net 24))
 (segment (start 191.3 70.7) (end 190 72) (width 0.25) (layer B.Cu) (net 24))
 (segment (start 175.49936 72) (end 174.99936 71.5) (width 0.25) (layer B.Cu) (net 24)))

